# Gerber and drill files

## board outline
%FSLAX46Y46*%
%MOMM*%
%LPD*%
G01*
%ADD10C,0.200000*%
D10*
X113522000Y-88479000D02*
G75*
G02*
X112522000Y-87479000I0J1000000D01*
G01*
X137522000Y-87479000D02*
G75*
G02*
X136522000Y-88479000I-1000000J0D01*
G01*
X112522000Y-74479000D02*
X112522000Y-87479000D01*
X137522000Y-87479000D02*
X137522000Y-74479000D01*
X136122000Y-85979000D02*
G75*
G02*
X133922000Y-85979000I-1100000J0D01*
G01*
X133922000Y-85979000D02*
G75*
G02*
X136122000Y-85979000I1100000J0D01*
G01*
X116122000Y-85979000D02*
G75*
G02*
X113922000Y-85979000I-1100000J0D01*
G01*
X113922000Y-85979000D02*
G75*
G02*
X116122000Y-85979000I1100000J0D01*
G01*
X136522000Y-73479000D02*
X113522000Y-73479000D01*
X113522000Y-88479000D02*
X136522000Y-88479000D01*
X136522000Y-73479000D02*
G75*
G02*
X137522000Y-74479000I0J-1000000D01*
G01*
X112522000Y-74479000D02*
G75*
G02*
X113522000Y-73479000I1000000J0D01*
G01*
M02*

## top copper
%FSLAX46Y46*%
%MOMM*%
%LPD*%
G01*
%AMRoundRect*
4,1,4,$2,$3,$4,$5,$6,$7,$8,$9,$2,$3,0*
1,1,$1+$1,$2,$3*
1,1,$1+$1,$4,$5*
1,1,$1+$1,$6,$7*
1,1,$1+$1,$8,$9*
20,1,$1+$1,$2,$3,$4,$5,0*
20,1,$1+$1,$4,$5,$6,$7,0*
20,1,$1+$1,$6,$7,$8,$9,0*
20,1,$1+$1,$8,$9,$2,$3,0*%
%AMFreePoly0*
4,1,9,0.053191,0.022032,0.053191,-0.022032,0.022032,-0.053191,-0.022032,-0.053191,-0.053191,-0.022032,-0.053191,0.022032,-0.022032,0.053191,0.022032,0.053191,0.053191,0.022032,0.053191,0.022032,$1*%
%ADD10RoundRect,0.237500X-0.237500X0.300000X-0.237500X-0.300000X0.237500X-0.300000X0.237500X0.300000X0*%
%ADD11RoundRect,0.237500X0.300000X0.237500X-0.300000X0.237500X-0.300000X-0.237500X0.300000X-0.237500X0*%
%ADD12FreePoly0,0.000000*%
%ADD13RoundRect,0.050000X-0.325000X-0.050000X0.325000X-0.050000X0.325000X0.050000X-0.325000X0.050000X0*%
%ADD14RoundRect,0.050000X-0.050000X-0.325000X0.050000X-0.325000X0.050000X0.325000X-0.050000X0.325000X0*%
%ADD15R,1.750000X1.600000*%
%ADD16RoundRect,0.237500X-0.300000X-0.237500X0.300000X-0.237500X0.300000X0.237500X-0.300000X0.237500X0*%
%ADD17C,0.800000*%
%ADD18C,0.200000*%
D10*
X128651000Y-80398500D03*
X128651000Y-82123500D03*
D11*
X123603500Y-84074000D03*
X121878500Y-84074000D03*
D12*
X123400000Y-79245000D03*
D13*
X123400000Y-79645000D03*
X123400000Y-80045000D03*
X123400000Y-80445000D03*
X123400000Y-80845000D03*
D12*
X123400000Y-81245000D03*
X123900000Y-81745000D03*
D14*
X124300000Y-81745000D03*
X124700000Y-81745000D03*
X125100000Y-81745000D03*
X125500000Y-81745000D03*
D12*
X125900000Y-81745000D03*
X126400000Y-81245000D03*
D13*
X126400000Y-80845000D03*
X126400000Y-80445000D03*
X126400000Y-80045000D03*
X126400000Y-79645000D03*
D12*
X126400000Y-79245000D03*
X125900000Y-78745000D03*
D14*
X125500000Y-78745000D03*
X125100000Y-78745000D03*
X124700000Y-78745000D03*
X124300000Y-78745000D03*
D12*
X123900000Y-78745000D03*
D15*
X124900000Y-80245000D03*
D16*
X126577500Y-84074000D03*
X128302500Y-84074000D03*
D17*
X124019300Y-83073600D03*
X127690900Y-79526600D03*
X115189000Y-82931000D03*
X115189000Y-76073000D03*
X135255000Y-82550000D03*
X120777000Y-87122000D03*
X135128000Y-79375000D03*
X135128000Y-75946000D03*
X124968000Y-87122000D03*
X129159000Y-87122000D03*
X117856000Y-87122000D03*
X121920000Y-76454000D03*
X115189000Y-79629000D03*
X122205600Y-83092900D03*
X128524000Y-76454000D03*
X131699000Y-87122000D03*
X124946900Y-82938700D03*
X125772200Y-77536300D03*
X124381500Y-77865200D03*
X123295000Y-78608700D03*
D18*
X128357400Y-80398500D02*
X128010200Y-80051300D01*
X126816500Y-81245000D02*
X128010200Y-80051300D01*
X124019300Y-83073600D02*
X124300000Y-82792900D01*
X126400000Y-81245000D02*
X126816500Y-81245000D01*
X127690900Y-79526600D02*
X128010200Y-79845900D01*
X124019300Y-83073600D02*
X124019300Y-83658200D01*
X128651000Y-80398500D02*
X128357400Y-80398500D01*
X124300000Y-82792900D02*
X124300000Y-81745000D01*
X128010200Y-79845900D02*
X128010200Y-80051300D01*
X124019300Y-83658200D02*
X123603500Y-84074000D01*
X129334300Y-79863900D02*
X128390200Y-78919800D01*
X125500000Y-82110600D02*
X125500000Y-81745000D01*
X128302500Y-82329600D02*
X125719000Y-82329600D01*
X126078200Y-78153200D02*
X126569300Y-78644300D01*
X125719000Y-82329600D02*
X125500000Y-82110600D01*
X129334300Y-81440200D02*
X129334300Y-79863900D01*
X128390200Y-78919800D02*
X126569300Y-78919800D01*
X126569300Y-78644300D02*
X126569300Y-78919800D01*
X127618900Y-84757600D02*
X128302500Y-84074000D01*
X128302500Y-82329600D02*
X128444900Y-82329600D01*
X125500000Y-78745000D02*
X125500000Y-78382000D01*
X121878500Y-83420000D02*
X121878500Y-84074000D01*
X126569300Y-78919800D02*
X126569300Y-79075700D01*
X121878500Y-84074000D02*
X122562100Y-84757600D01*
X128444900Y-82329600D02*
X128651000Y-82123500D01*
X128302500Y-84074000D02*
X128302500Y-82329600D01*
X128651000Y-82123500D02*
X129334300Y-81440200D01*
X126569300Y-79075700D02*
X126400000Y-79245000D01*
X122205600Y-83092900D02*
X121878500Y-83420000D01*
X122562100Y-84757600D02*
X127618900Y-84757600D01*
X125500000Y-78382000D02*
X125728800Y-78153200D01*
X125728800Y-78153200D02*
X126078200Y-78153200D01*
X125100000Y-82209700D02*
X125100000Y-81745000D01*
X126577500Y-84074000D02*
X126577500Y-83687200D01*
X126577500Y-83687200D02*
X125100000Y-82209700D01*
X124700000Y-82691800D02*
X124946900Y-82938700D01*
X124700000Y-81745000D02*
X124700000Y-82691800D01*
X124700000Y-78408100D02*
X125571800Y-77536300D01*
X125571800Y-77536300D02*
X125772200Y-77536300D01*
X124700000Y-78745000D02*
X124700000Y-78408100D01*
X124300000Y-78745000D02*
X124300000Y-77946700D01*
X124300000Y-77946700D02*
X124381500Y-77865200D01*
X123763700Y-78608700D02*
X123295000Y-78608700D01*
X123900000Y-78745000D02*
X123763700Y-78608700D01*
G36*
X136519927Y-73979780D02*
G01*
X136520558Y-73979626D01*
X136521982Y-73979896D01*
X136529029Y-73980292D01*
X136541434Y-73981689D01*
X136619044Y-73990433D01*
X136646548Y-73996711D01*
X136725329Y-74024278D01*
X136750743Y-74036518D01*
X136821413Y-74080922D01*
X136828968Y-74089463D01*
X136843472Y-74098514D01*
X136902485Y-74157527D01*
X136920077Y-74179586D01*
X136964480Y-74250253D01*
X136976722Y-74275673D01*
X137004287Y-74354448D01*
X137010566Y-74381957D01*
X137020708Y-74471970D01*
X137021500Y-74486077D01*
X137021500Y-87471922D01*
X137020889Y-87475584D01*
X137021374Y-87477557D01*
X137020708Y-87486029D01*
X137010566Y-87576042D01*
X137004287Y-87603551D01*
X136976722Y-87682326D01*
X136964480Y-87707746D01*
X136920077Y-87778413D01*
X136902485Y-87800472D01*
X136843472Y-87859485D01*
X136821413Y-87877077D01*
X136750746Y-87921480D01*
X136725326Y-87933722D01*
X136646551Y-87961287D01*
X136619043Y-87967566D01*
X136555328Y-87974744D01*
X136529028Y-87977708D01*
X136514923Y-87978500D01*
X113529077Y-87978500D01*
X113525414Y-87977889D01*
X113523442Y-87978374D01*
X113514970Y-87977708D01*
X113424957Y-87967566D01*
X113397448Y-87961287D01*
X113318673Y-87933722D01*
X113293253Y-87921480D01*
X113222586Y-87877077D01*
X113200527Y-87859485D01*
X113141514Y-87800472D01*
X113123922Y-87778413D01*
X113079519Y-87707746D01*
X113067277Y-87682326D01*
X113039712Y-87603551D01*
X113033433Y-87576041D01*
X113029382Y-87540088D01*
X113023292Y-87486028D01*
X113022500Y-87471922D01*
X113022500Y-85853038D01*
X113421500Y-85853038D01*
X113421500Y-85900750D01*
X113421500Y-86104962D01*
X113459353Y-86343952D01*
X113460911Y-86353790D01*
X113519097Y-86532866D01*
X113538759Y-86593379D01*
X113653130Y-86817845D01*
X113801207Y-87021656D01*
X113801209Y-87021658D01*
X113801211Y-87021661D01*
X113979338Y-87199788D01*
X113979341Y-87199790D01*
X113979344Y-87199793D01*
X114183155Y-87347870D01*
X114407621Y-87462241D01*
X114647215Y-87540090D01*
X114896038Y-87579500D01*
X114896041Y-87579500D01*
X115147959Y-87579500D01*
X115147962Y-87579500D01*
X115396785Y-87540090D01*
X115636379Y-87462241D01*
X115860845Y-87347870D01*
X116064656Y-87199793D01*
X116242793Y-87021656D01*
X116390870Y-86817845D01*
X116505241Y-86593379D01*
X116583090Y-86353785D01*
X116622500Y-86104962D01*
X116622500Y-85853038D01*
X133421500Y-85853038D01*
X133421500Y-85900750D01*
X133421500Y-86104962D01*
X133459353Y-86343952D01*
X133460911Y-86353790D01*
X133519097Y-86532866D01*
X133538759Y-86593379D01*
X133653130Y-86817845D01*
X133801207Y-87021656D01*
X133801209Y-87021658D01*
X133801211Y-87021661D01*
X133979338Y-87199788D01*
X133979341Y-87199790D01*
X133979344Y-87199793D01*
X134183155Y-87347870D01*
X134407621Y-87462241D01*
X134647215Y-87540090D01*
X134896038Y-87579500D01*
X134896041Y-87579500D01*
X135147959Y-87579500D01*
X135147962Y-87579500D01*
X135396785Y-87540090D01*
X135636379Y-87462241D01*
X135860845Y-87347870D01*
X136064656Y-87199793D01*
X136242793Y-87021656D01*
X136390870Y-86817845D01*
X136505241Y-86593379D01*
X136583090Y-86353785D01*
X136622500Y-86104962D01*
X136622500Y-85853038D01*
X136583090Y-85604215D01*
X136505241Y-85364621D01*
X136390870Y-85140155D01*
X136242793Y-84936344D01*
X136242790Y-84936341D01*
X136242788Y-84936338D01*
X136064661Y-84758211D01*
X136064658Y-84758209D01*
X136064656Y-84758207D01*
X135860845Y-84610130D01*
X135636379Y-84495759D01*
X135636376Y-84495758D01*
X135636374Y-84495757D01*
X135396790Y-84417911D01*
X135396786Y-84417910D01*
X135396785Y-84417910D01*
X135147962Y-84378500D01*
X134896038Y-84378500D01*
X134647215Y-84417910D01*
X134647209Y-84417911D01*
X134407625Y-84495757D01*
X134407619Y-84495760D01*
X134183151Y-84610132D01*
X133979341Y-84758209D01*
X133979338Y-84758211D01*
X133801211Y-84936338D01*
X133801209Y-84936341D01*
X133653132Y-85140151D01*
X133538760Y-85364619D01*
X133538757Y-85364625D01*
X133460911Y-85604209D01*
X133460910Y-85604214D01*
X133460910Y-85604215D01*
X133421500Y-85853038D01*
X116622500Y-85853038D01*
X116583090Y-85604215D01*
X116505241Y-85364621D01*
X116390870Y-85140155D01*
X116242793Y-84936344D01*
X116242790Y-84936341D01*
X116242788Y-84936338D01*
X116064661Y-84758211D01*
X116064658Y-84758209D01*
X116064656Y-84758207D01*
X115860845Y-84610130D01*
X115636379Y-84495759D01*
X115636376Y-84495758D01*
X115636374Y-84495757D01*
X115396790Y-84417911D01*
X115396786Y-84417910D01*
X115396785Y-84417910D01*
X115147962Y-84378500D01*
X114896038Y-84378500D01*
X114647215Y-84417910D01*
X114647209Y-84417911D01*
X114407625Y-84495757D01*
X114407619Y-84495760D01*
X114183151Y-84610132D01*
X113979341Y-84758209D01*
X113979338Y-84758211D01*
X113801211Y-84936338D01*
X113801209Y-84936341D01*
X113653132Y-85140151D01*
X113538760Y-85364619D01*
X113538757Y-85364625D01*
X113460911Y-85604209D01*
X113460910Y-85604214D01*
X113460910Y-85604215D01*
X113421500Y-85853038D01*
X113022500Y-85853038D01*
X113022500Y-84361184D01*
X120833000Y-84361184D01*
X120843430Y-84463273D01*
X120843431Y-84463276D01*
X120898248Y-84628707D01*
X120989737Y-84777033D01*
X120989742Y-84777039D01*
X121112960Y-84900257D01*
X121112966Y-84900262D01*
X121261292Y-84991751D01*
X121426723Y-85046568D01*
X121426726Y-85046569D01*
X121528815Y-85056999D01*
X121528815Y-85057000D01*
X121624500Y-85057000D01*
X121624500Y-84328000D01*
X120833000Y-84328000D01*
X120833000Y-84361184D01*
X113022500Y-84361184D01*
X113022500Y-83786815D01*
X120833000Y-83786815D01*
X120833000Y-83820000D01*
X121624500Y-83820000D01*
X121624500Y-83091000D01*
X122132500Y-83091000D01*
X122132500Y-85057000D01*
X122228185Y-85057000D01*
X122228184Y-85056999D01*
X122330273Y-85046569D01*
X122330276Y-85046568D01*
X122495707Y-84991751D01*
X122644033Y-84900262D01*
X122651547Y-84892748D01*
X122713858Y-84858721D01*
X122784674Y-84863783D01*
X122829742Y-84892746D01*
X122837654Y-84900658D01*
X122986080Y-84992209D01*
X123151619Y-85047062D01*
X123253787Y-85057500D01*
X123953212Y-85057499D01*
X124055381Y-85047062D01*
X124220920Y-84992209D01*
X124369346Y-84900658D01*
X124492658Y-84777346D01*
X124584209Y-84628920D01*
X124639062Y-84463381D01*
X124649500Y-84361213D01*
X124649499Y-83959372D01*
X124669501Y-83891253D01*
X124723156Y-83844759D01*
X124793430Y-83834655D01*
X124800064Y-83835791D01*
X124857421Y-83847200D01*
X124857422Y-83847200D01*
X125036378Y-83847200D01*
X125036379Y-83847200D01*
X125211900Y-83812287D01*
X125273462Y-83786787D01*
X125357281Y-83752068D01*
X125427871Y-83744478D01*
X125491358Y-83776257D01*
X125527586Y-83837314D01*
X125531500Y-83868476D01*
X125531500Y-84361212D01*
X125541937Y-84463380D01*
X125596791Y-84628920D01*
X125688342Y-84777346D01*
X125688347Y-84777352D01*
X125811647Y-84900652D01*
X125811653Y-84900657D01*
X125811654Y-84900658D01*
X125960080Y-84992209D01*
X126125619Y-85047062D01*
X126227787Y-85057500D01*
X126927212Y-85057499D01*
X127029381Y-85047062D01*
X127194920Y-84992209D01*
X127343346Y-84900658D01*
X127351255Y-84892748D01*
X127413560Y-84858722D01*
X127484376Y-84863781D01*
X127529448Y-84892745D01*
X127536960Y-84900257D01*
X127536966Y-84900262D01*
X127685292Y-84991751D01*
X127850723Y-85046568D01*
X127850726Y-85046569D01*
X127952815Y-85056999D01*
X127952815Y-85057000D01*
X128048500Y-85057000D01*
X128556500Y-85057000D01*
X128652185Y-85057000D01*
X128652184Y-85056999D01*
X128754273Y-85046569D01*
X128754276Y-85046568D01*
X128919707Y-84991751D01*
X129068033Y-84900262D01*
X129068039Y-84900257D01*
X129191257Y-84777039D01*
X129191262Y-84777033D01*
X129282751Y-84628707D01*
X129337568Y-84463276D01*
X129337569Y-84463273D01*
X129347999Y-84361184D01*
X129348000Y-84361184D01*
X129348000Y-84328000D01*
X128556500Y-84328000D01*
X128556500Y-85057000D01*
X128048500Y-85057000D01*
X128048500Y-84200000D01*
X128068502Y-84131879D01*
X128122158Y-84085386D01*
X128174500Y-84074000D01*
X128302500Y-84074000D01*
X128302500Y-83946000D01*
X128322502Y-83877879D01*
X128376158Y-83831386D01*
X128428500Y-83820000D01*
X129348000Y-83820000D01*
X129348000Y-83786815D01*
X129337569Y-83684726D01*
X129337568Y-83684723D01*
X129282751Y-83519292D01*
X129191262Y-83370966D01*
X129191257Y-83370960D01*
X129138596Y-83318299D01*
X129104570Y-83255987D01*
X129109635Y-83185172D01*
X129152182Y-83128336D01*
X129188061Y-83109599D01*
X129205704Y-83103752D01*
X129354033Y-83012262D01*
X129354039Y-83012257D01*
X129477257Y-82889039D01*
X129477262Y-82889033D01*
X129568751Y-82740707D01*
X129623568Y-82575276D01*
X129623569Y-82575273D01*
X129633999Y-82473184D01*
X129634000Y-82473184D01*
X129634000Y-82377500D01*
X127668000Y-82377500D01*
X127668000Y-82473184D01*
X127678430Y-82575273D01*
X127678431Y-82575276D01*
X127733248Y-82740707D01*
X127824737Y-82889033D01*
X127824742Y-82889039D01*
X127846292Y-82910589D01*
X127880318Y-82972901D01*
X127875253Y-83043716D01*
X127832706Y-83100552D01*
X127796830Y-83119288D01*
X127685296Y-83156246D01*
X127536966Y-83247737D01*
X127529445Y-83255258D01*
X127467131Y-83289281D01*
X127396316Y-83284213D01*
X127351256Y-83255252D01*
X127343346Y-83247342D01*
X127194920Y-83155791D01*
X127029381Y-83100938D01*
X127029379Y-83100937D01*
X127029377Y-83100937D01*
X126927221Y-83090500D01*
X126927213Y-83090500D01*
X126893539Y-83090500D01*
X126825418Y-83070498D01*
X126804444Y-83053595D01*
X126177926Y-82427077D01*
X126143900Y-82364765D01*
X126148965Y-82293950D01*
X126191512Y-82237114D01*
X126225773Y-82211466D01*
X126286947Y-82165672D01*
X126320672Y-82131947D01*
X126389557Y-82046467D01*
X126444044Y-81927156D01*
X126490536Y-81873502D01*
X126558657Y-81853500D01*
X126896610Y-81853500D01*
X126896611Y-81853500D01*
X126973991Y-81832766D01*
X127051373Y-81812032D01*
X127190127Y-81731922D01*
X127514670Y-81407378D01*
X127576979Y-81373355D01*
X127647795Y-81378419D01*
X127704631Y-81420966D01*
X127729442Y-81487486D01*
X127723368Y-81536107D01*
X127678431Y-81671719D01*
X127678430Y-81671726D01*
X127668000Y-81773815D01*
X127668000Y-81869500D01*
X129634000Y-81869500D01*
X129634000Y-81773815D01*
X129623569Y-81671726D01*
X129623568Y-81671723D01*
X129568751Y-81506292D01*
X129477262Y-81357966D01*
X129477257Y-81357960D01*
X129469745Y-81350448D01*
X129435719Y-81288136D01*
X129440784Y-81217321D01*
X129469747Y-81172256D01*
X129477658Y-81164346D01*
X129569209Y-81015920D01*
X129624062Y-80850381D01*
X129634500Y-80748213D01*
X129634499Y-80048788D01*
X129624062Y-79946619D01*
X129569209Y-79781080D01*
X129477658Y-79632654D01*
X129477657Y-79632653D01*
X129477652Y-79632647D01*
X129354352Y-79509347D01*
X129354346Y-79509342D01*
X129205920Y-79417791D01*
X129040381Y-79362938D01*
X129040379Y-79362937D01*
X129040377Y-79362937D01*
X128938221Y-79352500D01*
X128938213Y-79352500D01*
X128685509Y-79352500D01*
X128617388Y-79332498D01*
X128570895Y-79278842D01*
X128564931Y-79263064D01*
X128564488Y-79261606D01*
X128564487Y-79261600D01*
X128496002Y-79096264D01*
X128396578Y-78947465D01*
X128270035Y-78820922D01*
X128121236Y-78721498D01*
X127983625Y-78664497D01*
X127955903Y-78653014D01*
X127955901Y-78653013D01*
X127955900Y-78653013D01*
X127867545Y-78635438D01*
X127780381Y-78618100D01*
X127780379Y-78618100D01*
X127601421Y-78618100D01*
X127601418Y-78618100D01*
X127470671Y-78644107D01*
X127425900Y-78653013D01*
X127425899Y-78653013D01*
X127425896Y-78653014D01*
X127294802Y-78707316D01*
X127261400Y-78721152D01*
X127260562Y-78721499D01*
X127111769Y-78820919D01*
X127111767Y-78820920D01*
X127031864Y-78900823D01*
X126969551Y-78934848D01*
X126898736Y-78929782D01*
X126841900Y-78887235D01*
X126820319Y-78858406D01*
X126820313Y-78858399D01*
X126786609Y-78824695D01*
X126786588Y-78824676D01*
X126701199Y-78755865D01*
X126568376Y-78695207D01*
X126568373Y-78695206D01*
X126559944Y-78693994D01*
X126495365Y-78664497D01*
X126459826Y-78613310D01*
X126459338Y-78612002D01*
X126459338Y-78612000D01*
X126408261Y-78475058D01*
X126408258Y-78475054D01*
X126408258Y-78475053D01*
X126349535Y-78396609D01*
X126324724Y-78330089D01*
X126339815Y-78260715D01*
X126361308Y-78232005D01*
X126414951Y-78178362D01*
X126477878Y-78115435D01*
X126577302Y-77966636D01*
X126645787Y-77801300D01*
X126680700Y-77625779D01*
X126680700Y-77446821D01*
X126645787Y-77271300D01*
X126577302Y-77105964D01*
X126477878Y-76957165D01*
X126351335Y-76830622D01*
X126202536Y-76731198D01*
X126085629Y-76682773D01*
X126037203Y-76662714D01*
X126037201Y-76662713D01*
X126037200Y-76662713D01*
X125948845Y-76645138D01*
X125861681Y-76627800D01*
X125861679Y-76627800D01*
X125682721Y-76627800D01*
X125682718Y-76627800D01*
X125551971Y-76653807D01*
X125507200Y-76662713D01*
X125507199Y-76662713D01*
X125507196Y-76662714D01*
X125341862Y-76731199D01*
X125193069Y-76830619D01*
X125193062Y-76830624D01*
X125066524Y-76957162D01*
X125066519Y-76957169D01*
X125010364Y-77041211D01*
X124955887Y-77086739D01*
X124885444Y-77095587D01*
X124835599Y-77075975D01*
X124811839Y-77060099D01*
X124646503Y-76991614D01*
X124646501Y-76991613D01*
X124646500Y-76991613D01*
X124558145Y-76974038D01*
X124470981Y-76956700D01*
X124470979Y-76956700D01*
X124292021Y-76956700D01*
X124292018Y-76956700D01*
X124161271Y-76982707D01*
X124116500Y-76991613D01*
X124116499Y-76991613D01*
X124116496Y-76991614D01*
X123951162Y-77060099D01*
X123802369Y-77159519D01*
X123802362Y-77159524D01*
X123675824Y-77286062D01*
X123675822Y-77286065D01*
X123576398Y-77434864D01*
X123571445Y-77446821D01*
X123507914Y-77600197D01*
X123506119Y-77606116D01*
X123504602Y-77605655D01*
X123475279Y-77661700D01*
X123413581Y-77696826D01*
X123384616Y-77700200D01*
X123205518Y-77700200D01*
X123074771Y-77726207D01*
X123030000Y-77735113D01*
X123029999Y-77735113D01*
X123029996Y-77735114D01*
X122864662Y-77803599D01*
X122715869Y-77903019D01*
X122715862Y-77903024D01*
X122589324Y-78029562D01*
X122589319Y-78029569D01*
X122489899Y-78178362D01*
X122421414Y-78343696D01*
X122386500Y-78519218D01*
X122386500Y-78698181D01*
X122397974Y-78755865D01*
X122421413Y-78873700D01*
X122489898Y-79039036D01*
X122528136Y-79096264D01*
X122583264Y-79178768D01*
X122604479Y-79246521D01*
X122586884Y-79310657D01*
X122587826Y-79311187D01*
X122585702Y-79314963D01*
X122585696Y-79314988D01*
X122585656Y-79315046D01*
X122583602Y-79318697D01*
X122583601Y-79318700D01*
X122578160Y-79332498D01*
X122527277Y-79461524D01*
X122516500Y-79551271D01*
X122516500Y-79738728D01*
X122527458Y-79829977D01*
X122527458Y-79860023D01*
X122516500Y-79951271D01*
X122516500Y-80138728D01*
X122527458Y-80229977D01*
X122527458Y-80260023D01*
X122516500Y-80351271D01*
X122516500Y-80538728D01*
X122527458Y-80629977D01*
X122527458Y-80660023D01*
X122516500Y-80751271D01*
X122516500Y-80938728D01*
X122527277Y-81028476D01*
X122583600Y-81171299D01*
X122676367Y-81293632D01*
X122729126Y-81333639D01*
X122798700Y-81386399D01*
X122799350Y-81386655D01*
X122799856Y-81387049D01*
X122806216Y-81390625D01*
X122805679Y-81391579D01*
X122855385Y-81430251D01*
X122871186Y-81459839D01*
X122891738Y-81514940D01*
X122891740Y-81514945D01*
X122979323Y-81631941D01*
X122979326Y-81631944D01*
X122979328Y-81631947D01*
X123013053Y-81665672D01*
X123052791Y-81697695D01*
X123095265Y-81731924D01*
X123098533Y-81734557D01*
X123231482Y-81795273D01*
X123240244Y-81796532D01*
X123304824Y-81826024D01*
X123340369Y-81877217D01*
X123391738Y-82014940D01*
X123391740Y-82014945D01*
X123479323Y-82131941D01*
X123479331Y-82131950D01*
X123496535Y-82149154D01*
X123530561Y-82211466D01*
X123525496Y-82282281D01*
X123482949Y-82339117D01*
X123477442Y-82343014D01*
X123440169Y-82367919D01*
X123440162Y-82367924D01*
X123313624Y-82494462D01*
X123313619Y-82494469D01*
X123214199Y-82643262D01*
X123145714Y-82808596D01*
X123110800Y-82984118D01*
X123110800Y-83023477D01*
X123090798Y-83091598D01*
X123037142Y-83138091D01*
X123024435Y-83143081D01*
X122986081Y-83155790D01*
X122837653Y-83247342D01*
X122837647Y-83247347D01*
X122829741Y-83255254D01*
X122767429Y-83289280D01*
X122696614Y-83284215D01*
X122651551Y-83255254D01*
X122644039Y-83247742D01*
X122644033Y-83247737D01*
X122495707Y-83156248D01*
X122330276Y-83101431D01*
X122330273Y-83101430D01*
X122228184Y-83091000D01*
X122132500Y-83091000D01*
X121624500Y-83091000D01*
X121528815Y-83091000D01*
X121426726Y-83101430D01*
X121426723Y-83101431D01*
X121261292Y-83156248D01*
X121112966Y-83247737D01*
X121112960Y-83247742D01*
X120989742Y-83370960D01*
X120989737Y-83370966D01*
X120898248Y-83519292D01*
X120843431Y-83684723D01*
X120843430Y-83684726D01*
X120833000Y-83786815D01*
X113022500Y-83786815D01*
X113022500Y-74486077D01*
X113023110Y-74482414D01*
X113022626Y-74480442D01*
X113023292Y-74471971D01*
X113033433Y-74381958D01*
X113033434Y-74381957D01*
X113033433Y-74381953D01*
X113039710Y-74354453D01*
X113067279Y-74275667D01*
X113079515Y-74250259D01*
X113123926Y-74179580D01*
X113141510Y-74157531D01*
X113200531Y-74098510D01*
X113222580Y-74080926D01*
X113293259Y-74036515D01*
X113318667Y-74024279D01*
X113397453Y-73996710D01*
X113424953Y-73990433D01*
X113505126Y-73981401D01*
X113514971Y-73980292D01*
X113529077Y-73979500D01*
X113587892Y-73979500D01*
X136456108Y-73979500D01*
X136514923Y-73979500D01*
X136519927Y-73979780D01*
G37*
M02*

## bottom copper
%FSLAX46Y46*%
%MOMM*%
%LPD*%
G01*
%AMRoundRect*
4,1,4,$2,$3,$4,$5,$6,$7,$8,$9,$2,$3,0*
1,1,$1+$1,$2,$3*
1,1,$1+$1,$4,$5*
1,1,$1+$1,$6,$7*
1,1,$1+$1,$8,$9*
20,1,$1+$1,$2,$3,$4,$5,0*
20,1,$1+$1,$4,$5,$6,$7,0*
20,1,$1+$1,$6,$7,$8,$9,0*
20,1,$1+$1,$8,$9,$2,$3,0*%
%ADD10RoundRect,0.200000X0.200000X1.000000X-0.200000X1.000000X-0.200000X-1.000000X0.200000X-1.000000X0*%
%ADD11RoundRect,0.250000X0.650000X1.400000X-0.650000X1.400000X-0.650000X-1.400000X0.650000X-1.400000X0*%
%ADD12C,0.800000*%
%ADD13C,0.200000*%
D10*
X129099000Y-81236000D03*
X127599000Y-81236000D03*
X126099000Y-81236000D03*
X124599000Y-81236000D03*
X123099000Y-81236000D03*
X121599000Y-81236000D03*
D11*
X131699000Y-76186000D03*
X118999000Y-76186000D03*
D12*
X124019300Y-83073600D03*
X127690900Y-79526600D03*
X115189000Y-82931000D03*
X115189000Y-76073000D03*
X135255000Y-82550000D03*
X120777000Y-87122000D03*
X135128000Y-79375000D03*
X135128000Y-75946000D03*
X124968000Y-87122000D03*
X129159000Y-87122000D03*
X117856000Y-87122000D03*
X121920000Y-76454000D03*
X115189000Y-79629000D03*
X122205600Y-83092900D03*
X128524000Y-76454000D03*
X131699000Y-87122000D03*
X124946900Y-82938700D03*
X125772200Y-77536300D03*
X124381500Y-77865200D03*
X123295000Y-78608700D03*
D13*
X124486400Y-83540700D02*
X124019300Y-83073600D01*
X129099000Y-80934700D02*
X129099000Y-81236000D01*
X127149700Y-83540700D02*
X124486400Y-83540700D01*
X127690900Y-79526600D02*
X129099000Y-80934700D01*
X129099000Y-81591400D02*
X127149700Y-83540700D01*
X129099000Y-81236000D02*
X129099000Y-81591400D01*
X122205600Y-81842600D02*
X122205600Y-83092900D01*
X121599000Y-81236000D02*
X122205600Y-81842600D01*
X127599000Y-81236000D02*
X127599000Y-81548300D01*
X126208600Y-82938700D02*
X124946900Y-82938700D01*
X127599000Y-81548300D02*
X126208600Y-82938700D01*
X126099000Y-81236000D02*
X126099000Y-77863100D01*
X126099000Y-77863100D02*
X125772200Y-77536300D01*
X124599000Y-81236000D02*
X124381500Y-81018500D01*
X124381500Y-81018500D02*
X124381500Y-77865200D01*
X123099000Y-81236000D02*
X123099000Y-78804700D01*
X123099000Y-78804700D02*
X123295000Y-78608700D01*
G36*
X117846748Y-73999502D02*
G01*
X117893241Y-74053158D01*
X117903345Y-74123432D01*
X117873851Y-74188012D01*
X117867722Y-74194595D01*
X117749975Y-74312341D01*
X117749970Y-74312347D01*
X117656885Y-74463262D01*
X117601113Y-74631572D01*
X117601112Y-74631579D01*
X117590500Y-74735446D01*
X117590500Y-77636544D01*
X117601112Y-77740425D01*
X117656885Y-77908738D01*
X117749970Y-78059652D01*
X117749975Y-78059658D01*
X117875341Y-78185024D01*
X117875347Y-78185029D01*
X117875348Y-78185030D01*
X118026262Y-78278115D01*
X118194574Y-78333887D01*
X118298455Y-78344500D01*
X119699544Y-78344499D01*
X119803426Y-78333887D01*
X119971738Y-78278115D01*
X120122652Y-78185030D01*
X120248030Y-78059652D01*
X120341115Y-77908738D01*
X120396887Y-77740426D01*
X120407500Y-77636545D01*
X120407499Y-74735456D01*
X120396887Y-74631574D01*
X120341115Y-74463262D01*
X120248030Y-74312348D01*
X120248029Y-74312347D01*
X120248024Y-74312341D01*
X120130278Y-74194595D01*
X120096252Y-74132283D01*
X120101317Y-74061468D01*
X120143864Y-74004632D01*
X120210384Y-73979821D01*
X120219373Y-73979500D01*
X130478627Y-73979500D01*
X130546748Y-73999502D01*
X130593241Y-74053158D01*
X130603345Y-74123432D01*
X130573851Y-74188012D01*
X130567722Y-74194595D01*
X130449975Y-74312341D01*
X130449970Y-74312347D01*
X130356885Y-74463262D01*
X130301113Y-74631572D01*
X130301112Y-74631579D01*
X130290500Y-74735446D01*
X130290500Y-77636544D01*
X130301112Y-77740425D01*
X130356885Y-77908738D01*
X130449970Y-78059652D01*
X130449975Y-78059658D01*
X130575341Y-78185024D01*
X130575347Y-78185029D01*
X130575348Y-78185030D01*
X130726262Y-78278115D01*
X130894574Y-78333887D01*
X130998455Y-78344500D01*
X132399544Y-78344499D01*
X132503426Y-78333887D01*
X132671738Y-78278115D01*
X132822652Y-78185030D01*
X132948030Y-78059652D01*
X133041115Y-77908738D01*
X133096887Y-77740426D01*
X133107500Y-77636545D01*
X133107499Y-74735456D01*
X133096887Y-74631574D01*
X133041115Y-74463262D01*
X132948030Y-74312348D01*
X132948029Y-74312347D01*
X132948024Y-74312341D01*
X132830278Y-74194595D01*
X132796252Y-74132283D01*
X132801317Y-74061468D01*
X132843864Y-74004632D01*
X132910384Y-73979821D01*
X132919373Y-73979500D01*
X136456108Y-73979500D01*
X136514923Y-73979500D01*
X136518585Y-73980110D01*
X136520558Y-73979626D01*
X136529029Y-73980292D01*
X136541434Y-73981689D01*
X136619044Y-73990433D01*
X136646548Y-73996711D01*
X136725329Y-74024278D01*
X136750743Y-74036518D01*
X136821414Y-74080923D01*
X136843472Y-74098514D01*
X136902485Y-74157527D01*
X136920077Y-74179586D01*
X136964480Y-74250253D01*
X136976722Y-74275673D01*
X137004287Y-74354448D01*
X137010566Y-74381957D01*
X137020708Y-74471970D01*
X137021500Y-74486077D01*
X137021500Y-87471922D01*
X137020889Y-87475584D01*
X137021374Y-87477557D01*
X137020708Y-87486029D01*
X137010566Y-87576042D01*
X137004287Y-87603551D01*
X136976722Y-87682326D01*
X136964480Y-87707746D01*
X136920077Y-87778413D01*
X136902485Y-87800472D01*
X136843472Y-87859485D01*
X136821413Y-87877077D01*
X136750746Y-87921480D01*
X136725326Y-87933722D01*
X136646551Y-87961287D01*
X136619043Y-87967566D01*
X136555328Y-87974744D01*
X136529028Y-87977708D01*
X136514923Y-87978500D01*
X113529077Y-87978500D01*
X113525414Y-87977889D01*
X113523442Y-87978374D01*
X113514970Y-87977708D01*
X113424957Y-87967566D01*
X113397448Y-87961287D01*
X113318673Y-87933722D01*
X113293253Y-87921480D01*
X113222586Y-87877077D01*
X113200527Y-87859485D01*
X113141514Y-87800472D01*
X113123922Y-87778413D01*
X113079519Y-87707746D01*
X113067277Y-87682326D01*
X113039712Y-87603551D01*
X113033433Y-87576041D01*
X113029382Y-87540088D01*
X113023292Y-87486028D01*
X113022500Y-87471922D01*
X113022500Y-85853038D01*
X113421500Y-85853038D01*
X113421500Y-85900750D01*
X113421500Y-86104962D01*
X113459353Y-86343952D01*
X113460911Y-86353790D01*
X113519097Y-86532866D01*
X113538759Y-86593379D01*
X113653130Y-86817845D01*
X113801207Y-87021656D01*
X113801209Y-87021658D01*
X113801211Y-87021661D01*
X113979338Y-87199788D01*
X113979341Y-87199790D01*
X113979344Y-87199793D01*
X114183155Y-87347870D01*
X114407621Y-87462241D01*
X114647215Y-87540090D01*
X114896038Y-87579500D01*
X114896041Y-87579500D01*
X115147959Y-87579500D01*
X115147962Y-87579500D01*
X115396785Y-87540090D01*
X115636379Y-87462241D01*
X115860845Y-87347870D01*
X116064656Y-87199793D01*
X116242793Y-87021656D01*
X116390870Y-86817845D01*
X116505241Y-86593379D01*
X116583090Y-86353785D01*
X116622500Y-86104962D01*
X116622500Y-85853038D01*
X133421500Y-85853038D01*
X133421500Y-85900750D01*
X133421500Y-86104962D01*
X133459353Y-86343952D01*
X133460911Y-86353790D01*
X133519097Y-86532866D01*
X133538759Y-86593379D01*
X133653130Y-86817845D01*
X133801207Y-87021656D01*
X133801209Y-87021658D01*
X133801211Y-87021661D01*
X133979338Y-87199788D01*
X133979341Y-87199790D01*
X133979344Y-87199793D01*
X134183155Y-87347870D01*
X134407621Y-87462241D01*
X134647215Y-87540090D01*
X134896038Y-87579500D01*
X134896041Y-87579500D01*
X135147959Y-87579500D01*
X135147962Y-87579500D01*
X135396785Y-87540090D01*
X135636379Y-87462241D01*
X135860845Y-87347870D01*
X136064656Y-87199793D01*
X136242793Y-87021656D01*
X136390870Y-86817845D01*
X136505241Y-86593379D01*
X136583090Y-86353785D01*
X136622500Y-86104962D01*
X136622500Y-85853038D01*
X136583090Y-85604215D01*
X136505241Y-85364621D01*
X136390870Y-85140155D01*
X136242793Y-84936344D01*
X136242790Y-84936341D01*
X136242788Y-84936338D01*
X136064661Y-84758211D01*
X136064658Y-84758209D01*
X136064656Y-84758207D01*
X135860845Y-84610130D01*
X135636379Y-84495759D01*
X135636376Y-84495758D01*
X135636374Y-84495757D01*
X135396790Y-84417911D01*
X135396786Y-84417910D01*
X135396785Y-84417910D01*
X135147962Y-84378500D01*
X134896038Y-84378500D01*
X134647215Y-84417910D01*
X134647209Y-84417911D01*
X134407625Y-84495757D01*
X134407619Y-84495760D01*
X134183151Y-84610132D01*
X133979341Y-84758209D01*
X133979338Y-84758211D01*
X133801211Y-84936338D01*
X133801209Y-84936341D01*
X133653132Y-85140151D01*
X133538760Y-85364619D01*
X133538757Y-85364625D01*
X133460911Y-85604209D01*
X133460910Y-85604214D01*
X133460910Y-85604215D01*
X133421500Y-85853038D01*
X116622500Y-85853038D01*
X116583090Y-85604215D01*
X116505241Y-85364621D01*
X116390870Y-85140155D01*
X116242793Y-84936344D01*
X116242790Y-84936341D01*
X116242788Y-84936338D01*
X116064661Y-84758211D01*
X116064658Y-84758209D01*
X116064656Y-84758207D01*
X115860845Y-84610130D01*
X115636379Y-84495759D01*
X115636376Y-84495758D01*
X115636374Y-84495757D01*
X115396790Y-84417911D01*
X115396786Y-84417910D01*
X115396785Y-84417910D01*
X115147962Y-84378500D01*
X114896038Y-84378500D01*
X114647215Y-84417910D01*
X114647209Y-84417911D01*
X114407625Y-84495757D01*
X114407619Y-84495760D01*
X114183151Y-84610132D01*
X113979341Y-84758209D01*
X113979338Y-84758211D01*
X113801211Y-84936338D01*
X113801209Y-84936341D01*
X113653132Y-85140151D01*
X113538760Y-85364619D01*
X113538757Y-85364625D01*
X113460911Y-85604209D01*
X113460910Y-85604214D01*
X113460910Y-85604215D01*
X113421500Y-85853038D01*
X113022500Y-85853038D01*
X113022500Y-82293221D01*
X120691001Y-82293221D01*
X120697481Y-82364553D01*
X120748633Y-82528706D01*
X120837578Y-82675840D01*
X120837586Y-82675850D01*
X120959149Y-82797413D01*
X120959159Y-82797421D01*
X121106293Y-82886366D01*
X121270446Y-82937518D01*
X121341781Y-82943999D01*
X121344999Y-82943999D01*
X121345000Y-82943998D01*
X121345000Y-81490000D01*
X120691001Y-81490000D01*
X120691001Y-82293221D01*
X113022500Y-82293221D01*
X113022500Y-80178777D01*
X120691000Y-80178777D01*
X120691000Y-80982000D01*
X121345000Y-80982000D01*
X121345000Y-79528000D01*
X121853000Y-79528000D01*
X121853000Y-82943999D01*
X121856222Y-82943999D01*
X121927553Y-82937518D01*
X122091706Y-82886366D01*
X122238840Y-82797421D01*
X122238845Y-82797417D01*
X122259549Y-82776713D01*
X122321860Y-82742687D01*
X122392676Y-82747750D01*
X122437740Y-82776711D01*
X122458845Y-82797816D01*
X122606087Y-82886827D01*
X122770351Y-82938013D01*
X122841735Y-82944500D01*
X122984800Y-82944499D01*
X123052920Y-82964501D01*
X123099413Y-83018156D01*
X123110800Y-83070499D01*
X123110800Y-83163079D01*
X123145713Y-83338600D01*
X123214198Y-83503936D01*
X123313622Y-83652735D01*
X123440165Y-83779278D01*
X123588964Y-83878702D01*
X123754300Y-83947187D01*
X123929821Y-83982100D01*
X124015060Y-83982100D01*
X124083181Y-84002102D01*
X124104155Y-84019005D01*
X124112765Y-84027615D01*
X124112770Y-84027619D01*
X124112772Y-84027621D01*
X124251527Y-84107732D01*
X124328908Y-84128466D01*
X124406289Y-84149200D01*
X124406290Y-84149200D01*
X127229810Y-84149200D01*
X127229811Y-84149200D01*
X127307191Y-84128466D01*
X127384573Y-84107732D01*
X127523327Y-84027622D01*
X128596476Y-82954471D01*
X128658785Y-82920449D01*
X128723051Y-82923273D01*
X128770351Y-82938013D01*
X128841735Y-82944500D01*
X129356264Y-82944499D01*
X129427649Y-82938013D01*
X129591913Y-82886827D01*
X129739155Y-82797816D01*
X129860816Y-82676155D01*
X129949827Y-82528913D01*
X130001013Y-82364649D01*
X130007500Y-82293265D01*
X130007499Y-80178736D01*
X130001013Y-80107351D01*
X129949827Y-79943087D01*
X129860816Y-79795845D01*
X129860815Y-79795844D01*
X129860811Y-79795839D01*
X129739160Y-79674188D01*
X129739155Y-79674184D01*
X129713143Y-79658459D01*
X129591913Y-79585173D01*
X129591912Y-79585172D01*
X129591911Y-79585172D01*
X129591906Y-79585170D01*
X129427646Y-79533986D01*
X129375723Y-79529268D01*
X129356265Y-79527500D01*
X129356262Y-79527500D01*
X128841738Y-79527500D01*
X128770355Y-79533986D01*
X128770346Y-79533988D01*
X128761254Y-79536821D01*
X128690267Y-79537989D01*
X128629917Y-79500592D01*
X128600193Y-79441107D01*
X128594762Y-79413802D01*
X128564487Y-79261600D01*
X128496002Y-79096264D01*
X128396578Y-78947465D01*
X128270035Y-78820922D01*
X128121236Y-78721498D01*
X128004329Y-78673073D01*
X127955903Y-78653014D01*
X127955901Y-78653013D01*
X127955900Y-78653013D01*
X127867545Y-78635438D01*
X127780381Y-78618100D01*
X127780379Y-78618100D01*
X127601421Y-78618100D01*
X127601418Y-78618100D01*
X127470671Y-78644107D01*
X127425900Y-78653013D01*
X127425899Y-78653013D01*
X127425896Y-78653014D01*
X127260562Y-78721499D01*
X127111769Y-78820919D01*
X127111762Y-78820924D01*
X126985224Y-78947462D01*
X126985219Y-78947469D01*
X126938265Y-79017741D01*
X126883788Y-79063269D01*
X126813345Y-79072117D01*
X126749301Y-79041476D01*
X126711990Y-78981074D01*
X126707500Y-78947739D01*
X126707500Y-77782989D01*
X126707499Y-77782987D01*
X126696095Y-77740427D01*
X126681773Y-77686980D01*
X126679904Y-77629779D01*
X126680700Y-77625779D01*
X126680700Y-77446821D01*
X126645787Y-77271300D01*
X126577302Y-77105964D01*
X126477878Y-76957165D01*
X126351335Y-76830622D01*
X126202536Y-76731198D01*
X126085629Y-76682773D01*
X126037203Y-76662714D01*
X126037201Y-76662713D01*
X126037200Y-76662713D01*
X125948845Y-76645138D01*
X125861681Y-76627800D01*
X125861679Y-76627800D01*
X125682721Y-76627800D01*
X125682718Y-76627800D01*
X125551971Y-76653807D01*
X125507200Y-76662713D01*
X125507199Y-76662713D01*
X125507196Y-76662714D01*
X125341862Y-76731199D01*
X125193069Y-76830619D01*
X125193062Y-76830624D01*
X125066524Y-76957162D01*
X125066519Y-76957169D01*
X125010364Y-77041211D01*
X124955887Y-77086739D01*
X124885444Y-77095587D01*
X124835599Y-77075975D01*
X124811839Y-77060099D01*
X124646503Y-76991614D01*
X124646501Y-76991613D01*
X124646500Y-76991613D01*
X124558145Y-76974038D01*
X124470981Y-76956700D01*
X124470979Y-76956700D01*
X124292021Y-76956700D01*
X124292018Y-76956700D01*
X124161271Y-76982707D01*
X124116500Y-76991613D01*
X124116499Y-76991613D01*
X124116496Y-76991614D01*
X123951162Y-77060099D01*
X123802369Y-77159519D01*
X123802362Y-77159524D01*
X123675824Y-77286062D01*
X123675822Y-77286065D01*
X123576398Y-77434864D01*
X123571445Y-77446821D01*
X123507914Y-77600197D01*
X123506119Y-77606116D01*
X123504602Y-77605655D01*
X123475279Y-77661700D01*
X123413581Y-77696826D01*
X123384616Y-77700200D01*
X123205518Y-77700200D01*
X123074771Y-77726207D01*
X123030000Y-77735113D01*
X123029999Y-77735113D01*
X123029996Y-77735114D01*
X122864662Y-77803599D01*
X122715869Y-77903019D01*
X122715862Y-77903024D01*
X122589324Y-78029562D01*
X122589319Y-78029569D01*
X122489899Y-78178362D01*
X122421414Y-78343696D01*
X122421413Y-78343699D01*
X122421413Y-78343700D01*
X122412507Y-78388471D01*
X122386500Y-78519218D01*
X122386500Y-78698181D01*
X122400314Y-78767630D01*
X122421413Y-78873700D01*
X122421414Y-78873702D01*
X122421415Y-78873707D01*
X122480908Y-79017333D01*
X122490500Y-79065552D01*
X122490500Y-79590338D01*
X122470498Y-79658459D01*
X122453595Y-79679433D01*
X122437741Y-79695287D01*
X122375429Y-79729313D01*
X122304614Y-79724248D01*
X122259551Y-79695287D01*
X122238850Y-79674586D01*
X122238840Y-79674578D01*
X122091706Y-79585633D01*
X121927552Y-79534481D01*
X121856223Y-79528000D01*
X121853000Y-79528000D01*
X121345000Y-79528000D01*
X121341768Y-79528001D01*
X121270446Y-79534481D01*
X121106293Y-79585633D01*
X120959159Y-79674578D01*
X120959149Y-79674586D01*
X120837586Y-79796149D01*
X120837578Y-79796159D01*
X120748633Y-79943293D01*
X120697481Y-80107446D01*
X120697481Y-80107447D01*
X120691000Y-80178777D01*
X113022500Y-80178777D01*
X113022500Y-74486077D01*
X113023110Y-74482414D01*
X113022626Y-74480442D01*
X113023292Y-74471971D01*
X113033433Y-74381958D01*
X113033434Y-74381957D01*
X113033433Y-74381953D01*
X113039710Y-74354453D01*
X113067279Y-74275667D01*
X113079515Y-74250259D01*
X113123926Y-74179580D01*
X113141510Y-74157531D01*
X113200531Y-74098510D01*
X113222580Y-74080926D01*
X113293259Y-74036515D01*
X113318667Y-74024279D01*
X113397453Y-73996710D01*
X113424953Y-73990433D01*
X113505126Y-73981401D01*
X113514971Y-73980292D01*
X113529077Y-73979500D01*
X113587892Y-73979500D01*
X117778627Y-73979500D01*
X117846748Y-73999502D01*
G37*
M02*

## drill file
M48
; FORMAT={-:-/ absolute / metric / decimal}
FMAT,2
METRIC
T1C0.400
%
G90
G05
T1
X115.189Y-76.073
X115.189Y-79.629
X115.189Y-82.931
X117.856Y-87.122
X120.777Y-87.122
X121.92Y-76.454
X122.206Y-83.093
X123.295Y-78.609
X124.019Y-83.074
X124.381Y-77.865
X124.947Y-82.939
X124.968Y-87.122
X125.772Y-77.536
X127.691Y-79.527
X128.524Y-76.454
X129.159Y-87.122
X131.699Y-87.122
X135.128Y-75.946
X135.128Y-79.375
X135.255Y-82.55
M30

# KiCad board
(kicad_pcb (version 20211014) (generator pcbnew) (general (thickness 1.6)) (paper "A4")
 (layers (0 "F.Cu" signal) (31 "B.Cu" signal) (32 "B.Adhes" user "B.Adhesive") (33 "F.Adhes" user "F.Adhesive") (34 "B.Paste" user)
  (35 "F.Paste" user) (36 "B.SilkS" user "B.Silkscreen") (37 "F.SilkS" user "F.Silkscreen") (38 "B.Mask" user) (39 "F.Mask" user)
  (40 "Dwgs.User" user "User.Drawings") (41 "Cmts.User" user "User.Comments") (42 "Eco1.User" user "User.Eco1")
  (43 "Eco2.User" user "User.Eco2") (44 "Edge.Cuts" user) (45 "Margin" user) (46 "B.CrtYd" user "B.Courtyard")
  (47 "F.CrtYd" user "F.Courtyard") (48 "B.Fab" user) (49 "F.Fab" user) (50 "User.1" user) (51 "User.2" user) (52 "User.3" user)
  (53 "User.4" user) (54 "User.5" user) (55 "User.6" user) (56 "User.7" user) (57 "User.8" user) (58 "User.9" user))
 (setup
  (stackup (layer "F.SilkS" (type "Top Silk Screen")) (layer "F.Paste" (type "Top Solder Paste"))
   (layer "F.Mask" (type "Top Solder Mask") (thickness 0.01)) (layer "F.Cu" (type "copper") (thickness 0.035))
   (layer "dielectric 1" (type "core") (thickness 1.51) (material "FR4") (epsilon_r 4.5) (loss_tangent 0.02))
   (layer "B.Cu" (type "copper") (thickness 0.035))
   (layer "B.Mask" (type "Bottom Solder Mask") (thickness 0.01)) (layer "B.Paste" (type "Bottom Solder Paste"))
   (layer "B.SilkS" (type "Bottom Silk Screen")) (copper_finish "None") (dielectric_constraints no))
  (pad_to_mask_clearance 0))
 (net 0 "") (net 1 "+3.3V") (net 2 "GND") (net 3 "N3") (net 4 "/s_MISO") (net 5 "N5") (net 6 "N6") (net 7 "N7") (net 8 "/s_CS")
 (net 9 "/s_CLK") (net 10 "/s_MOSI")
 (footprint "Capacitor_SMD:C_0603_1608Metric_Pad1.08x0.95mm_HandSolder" (layer "F.Cu") (at 128.651 81.261 -90)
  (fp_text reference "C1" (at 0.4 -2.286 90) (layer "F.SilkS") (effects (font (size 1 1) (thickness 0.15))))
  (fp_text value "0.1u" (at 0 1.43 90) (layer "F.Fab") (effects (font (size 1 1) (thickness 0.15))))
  (pad "1" smd roundrect (at -0.8625 0 270) (size 1.075 0.95) (layers "F.Cu" "F.Paste" "F.Mask") (roundrect_rratio 0.25) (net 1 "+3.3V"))
  (pad "2" smd roundrect (at 0.8625 0 270) (size 1.075 0.95) (layers "F.Cu" "F.Paste" "F.Mask") (roundrect_rratio 0.25) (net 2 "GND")))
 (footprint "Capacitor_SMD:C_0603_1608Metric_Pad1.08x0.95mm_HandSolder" (layer "F.Cu") (at 122.741 84.074 180)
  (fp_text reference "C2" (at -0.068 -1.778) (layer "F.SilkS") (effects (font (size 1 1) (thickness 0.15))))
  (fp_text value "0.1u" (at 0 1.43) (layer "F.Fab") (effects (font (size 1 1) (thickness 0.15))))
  (pad "1" smd roundrect (at -0.8625 0 180) (size 1.075 0.95) (layers "F.Cu" "F.Paste" "F.Mask") (roundrect_rratio 0.25) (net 1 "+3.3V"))
  (pad "2" smd roundrect (at 0.8625 0 180) (size 1.075 0.95) (layers "F.Cu" "F.Paste" "F.Mask") (roundrect_rratio 0.25) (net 2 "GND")))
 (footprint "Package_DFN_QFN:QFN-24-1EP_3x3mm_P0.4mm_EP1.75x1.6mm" (layer "F.Cu") (at 124.9 80.245)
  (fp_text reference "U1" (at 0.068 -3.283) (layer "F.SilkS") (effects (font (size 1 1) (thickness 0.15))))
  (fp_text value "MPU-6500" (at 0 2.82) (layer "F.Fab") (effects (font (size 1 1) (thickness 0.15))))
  (pad "" smd roundrect (at 0.44 0.4) (size 0.71 0.64) (layers "F.Paste") (roundrect_rratio 0.25))
  (pad "" smd roundrect (at -0.44 0.4) (size 0.71 0.64) (layers "F.Paste") (roundrect_rratio 0.25))
  (pad "" smd roundrect (at -0.44 -0.4) (size 0.71 0.64) (layers "F.Paste") (roundrect_rratio 0.25))
  (pad "" smd roundrect (at 0.44 -0.4) (size 0.71 0.64) (layers "F.Paste") (roundrect_rratio 0.25))
  (pad "1" smd custom (at -1.5 -1) (size 0.115147 0.115147) (layers "F.Cu" "F.Paste" "F.Mask") (options (clearance outline) (anchor circle))
   (primitives))
  (pad "2" smd roundrect (at -1.5 -0.6) (size 0.75 0.2) (layers "F.Cu" "F.Paste" "F.Mask") (roundrect_rratio 0.25))
  (pad "3" smd roundrect (at -1.5 -0.2) (size 0.75 0.2) (layers "F.Cu" "F.Paste" "F.Mask") (roundrect_rratio 0.25))
  (pad "4" smd roundrect (at -1.5 0.2) (size 0.75 0.2) (layers "F.Cu" "F.Paste" "F.Mask") (roundrect_rratio 0.25))
  (pad "5" smd roundrect (at -1.5 0.6) (size 0.75 0.2) (layers "F.Cu" "F.Paste" "F.Mask") (roundrect_rratio 0.25))
  (pad "6" smd custom (at -1.5 1) (size 0.115147 0.115147) (layers "F.Cu" "F.Paste" "F.Mask") (options (clearance outline) (anchor circle))
   (primitives))
  (pad "7" smd custom (at -1 1.5) (size 0.115147 0.115147) (layers "F.Cu" "F.Paste" "F.Mask") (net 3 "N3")
   (options (clearance outline) (anchor circle)) (primitives))
  (pad "8" smd roundrect (at -0.6 1.5) (size 0.2 0.75) (layers "F.Cu" "F.Paste" "F.Mask") (roundrect_rratio 0.25) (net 1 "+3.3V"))
  (pad "9" smd roundrect (at -0.2 1.5) (size 0.2 0.75) (layers "F.Cu" "F.Paste" "F.Mask") (roundrect_rratio 0.25) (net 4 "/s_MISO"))
  (pad "10" smd roundrect (at 0.2 1.5) (size 0.2 0.75) (layers "F.Cu" "F.Paste" "F.Mask") (roundrect_rratio 0.25) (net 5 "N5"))
  (pad "11" smd roundrect (at 0.6 1.5) (size 0.2 0.75) (layers "F.Cu" "F.Paste" "F.Mask") (roundrect_rratio 0.25) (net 2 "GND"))
  (pad "12" smd custom (at 1 1.5) (size 0.115147 0.115147) (layers "F.Cu" "F.Paste" "F.Mask") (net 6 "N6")
   (options (clearance outline) (anchor circle)) (primitives))
  (pad "13" smd custom (at 1.5 1) (size 0.115147 0.115147) (layers "F.Cu" "F.Paste" "F.Mask") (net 1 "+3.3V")
   (options (clearance outline) (anchor circle)) (primitives))
  (pad "14" smd roundrect (at 1.5 0.6) (size 0.75 0.2) (layers "F.Cu" "F.Paste" "F.Mask") (roundrect_rratio 0.25))
  (pad "15" smd roundrect (at 1.5 0.2) (size 0.75 0.2) (layers "F.Cu" "F.Paste" "F.Mask") (roundrect_rratio 0.25))
  (pad "16" smd roundrect (at 1.5 -0.2) (size 0.75 0.2) (layers "F.Cu" "F.Paste" "F.Mask") (roundrect_rratio 0.25))
  (pad "17" smd roundrect (at 1.5 -0.6) (size 0.75 0.2) (layers "F.Cu" "F.Paste" "F.Mask") (roundrect_rratio 0.25))
  (pad "18" smd custom (at 1.5 -1) (size 0.115147 0.115147) (layers "F.Cu" "F.Paste" "F.Mask") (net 2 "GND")
   (options (clearance outline) (anchor circle)) (primitives))
  (pad "19" smd custom (at 1 -1.5) (size 0.115147 0.115147) (layers "F.Cu" "F.Paste" "F.Mask") (options (clearance outline) (anchor circle))
   (primitives))
  (pad "20" smd roundrect (at 0.6 -1.5) (size 0.2 0.75) (layers "F.Cu" "F.Paste" "F.Mask") (roundrect_rratio 0.25) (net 2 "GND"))
  (pad "21" smd roundrect (at 0.2 -1.5) (size 0.2 0.75) (layers "F.Cu" "F.Paste" "F.Mask") (roundrect_rratio 0.25) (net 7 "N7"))
  (pad "22" smd roundrect (at -0.2 -1.5) (size 0.2 0.75) (layers "F.Cu" "F.Paste" "F.Mask") (roundrect_rratio 0.25) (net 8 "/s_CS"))
  (pad "23" smd roundrect (at -0.6 -1.5) (size 0.2 0.75) (layers "F.Cu" "F.Paste" "F.Mask") (roundrect_rratio 0.25) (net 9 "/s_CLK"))
  (pad "24" smd custom (at -1 -1.5) (size 0.115147 0.115147) (layers "F.Cu" "F.Paste" "F.Mask") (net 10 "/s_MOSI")
   (options (clearance outline) (anchor circle)) (primitives))
  (pad "25" smd rect (at 0 0) (size 1.75 1.6) (layers "F.Cu" "F.Mask")))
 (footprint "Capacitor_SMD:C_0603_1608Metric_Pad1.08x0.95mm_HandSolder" (layer "F.Cu") (at 127.44 84.074)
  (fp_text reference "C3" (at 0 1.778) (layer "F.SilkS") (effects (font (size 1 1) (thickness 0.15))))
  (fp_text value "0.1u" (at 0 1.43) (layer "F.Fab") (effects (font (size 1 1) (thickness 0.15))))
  (pad "1" smd roundrect (at -0.8625 0) (size 1.075 0.95) (layers "F.Cu" "F.Paste" "F.Mask") (roundrect_rratio 0.25) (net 5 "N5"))
  (pad "2" smd roundrect (at 0.8625 0) (size 1.075 0.95) (layers "F.Cu" "F.Paste" "F.Mask") (roundrect_rratio 0.25) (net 2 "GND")))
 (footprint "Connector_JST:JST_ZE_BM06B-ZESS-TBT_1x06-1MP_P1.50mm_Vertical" (layer "B.Cu") (at 125.349 78.486 180)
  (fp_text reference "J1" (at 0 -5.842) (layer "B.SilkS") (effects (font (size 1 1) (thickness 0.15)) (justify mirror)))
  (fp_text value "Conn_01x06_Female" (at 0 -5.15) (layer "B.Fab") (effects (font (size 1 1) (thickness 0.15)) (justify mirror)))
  (pad "1" smd roundrect (at -3.75 -2.75 180) (size 0.8 2.4) (layers "B.Cu" "B.Paste" "B.Mask") (roundrect_rratio 0.25) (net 1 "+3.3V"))
  (pad "2" smd roundrect (at -2.25 -2.75 180) (size 0.8 2.4) (layers "B.Cu" "B.Paste" "B.Mask") (roundrect_rratio 0.25) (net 4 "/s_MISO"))
  (pad "3" smd roundrect (at -0.75 -2.75 180) (size 0.8 2.4) (layers "B.Cu" "B.Paste" "B.Mask") (roundrect_rratio 0.25) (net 8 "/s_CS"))
  (pad "4" smd roundrect (at 0.75 -2.75 180) (size 0.8 2.4) (layers "B.Cu" "B.Paste" "B.Mask") (roundrect_rratio 0.25) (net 9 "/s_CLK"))
  (pad "5" smd roundrect (at 2.25 -2.75 180) (size 0.8 2.4) (layers "B.Cu" "B.Paste" "B.Mask") (roundrect_rratio 0.25) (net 10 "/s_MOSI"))
  (pad "6" smd roundrect (at 3.75 -2.75 180) (size 0.8 2.4) (layers "B.Cu" "B.Paste" "B.Mask") (roundrect_rratio 0.25) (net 2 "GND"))
  (pad "MP" smd roundrect (at -6.35 2.3 180) (size 1.8 3.3) (layers "B.Cu" "B.Paste" "B.Mask") (roundrect_rratio 0.138889))
  (pad "MP" smd roundrect (at 6.35 2.3 180) (size 1.8 3.3) (layers "B.Cu" "B.Paste" "B.Mask") (roundrect_rratio 0.138889)))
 (gr_arc (start 113.522 88.479) (mid 112.814893 88.186107) (end 112.522 87.479) (layer "Edge.Cuts") (width 0.2))
 (gr_arc (start 137.522 87.479) (mid 137.229107 88.186107) (end 136.522 88.479) (layer "Edge.Cuts") (width 0.2))
 (gr_line (start 112.522 74.479) (end 112.522 87.479) (layer "Edge.Cuts") (width 0.2))
 (gr_line (start 137.522 87.479) (end 137.522 74.479) (layer "Edge.Cuts") (width 0.2))
 (gr_circle (center 135.022 85.979) (end 135.022 87.079) (layer "Edge.Cuts") (width 0.2) (fill none))
 (gr_circle (center 115.022 85.979) (end 115.022 87.079) (layer "Edge.Cuts") (width 0.2) (fill none))
 (gr_line (start 136.522 73.479) (end 113.522 73.479) (layer "Edge.Cuts") (width 0.2))
 (gr_line (start 113.522 88.479) (end 136.522 88.479) (layer "Edge.Cuts") (width 0.2))
 (gr_arc (start 136.522 73.479) (mid 137.229107 73.771893) (end 137.522 74.479) (layer "Edge.Cuts") (width 0.2))
 (gr_arc (start 112.522 74.479) (mid 112.814893 73.771893) (end 113.522 73.479) (layer "Edge.Cuts") (width 0.2))
 (segment (start 128.3574 80.3985) (end 128.0102 80.0513) (width 0.2) (layer "F.Cu") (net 1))
 (segment (start 126.8165 81.245) (end 128.0102 80.0513) (width 0.2) (layer "F.Cu") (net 1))
 (segment (start 124.0193 83.0736) (end 124.3 82.7929) (width 0.2) (layer "F.Cu") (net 1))
 (segment (start 126.4 81.245) (end 126.8165 81.245) (width 0.2) (layer "F.Cu") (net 1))
 (segment (start 127.6909 79.5266) (end 128.0102 79.8459) (width 0.2) (layer "F.Cu") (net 1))
 (segment (start 124.0193 83.0736) (end 124.0193 83.6582) (width 0.2) (layer "F.Cu") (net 1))
 (segment (start 128.651 80.3985) (end 128.3574 80.3985) (width 0.2) (layer "F.Cu") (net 1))
 (segment (start 124.3 82.7929) (end 124.3 81.745) (width 0.2) (layer "F.Cu") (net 1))
 (segment (start 128.0102 79.8459) (end 128.0102 80.0513) (width 0.2) (layer "F.Cu") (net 1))
 (segment (start 124.0193 83.6582) (end 123.6035 84.074) (width 0.2) (layer "F.Cu") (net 1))
 (via (at 124.0193 83.0736) (size 0.8) (drill 0.4) (layers "F.Cu" "B.Cu") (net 1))
 (via (at 127.6909 79.5266) (size 0.8) (drill 0.4) (layers "F.Cu" "B.Cu") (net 1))
 (segment (start 124.4864 83.5407) (end 124.0193 83.0736) (width 0.2) (layer "B.Cu") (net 1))
 (segment (start 129.099 80.9347) (end 129.099 81.236) (width 0.2) (layer "B.Cu") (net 1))
 (segment (start 127.1497 83.5407) (end 124.4864 83.5407) (width 0.2) (layer "B.Cu") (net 1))
 (segment (start 127.6909 79.5266) (end 129.099 80.9347) (width 0.2) (layer "B.Cu") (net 1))
 (segment (start 129.099 81.5914) (end 127.1497 83.5407) (width 0.2) (layer "B.Cu") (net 1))
 (segment (start 129.099 81.236) (end 129.099 81.5914) (width 0.2) (layer "B.Cu") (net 1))
 (segment (start 129.3343 79.8639) (end 128.3902 78.9198) (width 0.2) (layer "F.Cu") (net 2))
 (segment (start 125.5 82.1106) (end 125.5 81.745) (width 0.2) (layer "F.Cu") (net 2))
 (segment (start 128.3025 82.3296) (end 125.719 82.3296) (width 0.2) (layer "F.Cu") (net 2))
 (segment (start 126.0782 78.1532) (end 126.5693 78.6443) (width 0.2) (layer "F.Cu") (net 2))
 (segment (start 125.719 82.3296) (end 125.5 82.1106) (width 0.2) (layer "F.Cu") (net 2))
 (segment (start 129.3343 81.4402) (end 129.3343 79.8639) (width 0.2) (layer "F.Cu") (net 2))
 (segment (start 128.3902 78.9198) (end 126.5693 78.9198) (width 0.2) (layer "F.Cu") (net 2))
 (segment (start 126.5693 78.6443) (end 126.5693 78.9198) (width 0.2) (layer "F.Cu") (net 2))
 (segment (start 127.6189 84.7576) (end 128.3025 84.074) (width 0.2) (layer "F.Cu") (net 2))
 (segment (start 128.3025 82.3296) (end 128.4449 82.3296) (width 0.2) (layer "F.Cu") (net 2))
 (segment (start 125.5 78.745) (end 125.5 78.382) (width 0.2) (layer "F.Cu") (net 2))
 (segment (start 121.8785 83.42) (end 121.8785 84.074) (width 0.2) (layer "F.Cu") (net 2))
 (segment (start 126.5693 78.9198) (end 126.5693 79.0757) (width 0.2) (layer "F.Cu") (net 2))
 (segment (start 121.8785 84.074) (end 122.5621 84.7576) (width 0.2) (layer "F.Cu") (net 2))
 (segment (start 128.4449 82.3296) (end 128.651 82.1235) (width 0.2) (layer "F.Cu") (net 2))
 (segment (start 128.3025 84.074) (end 128.3025 82.3296) (width 0.2) (layer "F.Cu") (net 2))
 (segment (start 128.651 82.1235) (end 129.3343 81.4402) (width 0.2) (layer "F.Cu") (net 2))
 (segment (start 126.5693 79.0757) (end 126.4 79.245) (width 0.2) (layer "F.Cu") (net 2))
 (segment (start 122.2056 83.0929) (end 121.8785 83.42) (width 0.2) (layer "F.Cu") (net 2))
 (segment (start 122.5621 84.7576) (end 127.6189 84.7576) (width 0.2) (layer "F.Cu") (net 2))
 (segment (start 125.5 78.382) (end 125.7288 78.1532) (width 0.2) (layer "F.Cu") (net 2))
 (segment (start 125.7288 78.1532) (end 126.0782 78.1532) (width 0.2) (layer "F.Cu") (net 2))
 (via (at 115.189 82.931) (size 0.8) (drill 0.4) (layers "F.Cu" "B.Cu") (free) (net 2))
 (via (at 115.189 76.073) (size 0.8) (drill 0.4) (layers "F.Cu" "B.Cu") (free) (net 2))
 (via (at 135.255 82.55) (size 0.8) (drill 0.4) (layers "F.Cu" "B.Cu") (free) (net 2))
 (via (at 120.777 87.122) (size 0.8) (drill 0.4) (layers "F.Cu" "B.Cu") (free) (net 2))
 (via (at 135.128 79.375) (size 0.8) (drill 0.4) (layers "F.Cu" "B.Cu") (free) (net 2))
 (via (at 135.128 75.946) (size 0.8) (drill 0.4) (layers "F.Cu" "B.Cu") (free) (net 2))
 (via (at 124.968 87.122) (size 0.8) (drill 0.4) (layers "F.Cu" "B.Cu") (free) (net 2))
 (via (at 129.159 87.122) (size 0.8) (drill 0.4) (layers "F.Cu" "B.Cu") (free) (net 2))
 (via (at 117.856 87.122) (size 0.8) (drill 0.4) (layers "F.Cu" "B.Cu") (free) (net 2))
 (via (at 121.92 76.454) (size 0.8) (drill 0.4) (layers "F.Cu" "B.Cu") (free) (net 2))
 (via (at 115.189 79.629) (size 0.8) (drill 0.4) (layers "F.Cu" "B.Cu") (free) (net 2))
 (via (at 122.2056 83.0929) (size 0.8) (drill 0.4) (layers "F.Cu" "B.Cu") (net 2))
 (via (at 128.524 76.454) (size 0.8) (drill 0.4) (layers "F.Cu" "B.Cu") (free) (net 2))
 (via (at 131.699 87.122) (size 0.8) (drill 0.4) (layers "F.Cu" "B.Cu") (free) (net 2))
 (segment (start 122.2056 81.8426) (end 122.2056 83.0929) (width 0.2) (layer "B.Cu") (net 2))
 (segment (start 121.599 81.236) (end 122.2056 81.8426) (width 0.2) (layer "B.Cu") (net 2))
 (segment (start 125.1 82.2097) (end 125.1 81.745) (width 0.2) (layer "F.Cu") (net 5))
 (segment (start 126.5775 84.074) (end 126.5775 83.6872) (width 0.2) (layer "F.Cu") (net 5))
 (segment (start 126.5775 83.6872) (end 125.1 82.2097) (width 0.2) (layer "F.Cu") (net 5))
 (segment (start 124.7 82.6918) (end 124.9469 82.9387) (width 0.2) (layer "F.Cu") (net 4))
 (segment (start 124.7 81.745) (end 124.7 82.6918) (width 0.2) (layer "F.Cu") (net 4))
 (via (at 124.9469 82.9387) (size 0.8) (drill 0.4) (layers "F.Cu" "B.Cu") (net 4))
 (segment (start 127.599 81.236) (end 127.599 81.5483) (width 0.2) (layer "B.Cu") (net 4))
 (segment (start 126.2086 82.9387) (end 124.9469 82.9387) (width 0.2) (layer "B.Cu") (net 4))
 (segment (start 127.599 81.5483) (end 126.2086 82.9387) (width 0.2) (layer "B.Cu") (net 4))
 (segment (start 124.7 78.4081) (end 125.5718 77.5363) (width 0.2) (layer "F.Cu") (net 8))
 (segment (start 125.5718 77.5363) (end 125.7722 77.5363) (width 0.2) (layer "F.Cu") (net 8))
 (segment (start 124.7 78.745) (end 124.7 78.4081) (width 0.2) (layer "F.Cu") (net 8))
 (via (at 125.7722 77.5363) (size 0.8) (drill 0.4) (layers "F.Cu" "B.Cu") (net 8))
 (segment (start 126.099 81.236) (end 126.099 77.8631) (width 0.2) (layer "B.Cu") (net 8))
 (segment (start 126.099 77.8631) (end 125.7722 77.5363) (width 0.2) (layer "B.Cu") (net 8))
 (segment (start 124.3 78.745) (end 124.3 77.9467) (width 0.2) (layer "F.Cu") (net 9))
 (segment (start 124.3 77.9467) (end 124.3815 77.8652) (width 0.2) (layer "F.Cu") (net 9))
 (via (at 124.3815 77.8652) (size 0.8) (drill 0.4) (layers "F.Cu" "B.Cu") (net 9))
 (segment (start 124.599 81.236) (end 124.3815 81.0185) (width 0.2) (layer "B.Cu") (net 9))
 (segment (start 124.3815 81.0185) (end 124.3815 77.8652) (width 0.2) (layer "B.Cu") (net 9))
 (segment (start 123.7637 78.6087) (end 123.295 78.6087) (width 0.2) (layer "F.Cu") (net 10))
 (segment (start 123.9 78.745) (end 123.7637 78.6087) (width 0.2) (layer "F.Cu") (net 10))
 (via (at 123.295 78.6087) (size 0.8) (drill 0.4) (layers "F.Cu" "B.Cu") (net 10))
 (segment (start 123.099 81.236) (end 123.099 78.8047) (width 0.2) (layer "B.Cu") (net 10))
 (segment (start 123.099 78.8047) (end 123.295 78.6087) (width 0.2) (layer "B.Cu") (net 10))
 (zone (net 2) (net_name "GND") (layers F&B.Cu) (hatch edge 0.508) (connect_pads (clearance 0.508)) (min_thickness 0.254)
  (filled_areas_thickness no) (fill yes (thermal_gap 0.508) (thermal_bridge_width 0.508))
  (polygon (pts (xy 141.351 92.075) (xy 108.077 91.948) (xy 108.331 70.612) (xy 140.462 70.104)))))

